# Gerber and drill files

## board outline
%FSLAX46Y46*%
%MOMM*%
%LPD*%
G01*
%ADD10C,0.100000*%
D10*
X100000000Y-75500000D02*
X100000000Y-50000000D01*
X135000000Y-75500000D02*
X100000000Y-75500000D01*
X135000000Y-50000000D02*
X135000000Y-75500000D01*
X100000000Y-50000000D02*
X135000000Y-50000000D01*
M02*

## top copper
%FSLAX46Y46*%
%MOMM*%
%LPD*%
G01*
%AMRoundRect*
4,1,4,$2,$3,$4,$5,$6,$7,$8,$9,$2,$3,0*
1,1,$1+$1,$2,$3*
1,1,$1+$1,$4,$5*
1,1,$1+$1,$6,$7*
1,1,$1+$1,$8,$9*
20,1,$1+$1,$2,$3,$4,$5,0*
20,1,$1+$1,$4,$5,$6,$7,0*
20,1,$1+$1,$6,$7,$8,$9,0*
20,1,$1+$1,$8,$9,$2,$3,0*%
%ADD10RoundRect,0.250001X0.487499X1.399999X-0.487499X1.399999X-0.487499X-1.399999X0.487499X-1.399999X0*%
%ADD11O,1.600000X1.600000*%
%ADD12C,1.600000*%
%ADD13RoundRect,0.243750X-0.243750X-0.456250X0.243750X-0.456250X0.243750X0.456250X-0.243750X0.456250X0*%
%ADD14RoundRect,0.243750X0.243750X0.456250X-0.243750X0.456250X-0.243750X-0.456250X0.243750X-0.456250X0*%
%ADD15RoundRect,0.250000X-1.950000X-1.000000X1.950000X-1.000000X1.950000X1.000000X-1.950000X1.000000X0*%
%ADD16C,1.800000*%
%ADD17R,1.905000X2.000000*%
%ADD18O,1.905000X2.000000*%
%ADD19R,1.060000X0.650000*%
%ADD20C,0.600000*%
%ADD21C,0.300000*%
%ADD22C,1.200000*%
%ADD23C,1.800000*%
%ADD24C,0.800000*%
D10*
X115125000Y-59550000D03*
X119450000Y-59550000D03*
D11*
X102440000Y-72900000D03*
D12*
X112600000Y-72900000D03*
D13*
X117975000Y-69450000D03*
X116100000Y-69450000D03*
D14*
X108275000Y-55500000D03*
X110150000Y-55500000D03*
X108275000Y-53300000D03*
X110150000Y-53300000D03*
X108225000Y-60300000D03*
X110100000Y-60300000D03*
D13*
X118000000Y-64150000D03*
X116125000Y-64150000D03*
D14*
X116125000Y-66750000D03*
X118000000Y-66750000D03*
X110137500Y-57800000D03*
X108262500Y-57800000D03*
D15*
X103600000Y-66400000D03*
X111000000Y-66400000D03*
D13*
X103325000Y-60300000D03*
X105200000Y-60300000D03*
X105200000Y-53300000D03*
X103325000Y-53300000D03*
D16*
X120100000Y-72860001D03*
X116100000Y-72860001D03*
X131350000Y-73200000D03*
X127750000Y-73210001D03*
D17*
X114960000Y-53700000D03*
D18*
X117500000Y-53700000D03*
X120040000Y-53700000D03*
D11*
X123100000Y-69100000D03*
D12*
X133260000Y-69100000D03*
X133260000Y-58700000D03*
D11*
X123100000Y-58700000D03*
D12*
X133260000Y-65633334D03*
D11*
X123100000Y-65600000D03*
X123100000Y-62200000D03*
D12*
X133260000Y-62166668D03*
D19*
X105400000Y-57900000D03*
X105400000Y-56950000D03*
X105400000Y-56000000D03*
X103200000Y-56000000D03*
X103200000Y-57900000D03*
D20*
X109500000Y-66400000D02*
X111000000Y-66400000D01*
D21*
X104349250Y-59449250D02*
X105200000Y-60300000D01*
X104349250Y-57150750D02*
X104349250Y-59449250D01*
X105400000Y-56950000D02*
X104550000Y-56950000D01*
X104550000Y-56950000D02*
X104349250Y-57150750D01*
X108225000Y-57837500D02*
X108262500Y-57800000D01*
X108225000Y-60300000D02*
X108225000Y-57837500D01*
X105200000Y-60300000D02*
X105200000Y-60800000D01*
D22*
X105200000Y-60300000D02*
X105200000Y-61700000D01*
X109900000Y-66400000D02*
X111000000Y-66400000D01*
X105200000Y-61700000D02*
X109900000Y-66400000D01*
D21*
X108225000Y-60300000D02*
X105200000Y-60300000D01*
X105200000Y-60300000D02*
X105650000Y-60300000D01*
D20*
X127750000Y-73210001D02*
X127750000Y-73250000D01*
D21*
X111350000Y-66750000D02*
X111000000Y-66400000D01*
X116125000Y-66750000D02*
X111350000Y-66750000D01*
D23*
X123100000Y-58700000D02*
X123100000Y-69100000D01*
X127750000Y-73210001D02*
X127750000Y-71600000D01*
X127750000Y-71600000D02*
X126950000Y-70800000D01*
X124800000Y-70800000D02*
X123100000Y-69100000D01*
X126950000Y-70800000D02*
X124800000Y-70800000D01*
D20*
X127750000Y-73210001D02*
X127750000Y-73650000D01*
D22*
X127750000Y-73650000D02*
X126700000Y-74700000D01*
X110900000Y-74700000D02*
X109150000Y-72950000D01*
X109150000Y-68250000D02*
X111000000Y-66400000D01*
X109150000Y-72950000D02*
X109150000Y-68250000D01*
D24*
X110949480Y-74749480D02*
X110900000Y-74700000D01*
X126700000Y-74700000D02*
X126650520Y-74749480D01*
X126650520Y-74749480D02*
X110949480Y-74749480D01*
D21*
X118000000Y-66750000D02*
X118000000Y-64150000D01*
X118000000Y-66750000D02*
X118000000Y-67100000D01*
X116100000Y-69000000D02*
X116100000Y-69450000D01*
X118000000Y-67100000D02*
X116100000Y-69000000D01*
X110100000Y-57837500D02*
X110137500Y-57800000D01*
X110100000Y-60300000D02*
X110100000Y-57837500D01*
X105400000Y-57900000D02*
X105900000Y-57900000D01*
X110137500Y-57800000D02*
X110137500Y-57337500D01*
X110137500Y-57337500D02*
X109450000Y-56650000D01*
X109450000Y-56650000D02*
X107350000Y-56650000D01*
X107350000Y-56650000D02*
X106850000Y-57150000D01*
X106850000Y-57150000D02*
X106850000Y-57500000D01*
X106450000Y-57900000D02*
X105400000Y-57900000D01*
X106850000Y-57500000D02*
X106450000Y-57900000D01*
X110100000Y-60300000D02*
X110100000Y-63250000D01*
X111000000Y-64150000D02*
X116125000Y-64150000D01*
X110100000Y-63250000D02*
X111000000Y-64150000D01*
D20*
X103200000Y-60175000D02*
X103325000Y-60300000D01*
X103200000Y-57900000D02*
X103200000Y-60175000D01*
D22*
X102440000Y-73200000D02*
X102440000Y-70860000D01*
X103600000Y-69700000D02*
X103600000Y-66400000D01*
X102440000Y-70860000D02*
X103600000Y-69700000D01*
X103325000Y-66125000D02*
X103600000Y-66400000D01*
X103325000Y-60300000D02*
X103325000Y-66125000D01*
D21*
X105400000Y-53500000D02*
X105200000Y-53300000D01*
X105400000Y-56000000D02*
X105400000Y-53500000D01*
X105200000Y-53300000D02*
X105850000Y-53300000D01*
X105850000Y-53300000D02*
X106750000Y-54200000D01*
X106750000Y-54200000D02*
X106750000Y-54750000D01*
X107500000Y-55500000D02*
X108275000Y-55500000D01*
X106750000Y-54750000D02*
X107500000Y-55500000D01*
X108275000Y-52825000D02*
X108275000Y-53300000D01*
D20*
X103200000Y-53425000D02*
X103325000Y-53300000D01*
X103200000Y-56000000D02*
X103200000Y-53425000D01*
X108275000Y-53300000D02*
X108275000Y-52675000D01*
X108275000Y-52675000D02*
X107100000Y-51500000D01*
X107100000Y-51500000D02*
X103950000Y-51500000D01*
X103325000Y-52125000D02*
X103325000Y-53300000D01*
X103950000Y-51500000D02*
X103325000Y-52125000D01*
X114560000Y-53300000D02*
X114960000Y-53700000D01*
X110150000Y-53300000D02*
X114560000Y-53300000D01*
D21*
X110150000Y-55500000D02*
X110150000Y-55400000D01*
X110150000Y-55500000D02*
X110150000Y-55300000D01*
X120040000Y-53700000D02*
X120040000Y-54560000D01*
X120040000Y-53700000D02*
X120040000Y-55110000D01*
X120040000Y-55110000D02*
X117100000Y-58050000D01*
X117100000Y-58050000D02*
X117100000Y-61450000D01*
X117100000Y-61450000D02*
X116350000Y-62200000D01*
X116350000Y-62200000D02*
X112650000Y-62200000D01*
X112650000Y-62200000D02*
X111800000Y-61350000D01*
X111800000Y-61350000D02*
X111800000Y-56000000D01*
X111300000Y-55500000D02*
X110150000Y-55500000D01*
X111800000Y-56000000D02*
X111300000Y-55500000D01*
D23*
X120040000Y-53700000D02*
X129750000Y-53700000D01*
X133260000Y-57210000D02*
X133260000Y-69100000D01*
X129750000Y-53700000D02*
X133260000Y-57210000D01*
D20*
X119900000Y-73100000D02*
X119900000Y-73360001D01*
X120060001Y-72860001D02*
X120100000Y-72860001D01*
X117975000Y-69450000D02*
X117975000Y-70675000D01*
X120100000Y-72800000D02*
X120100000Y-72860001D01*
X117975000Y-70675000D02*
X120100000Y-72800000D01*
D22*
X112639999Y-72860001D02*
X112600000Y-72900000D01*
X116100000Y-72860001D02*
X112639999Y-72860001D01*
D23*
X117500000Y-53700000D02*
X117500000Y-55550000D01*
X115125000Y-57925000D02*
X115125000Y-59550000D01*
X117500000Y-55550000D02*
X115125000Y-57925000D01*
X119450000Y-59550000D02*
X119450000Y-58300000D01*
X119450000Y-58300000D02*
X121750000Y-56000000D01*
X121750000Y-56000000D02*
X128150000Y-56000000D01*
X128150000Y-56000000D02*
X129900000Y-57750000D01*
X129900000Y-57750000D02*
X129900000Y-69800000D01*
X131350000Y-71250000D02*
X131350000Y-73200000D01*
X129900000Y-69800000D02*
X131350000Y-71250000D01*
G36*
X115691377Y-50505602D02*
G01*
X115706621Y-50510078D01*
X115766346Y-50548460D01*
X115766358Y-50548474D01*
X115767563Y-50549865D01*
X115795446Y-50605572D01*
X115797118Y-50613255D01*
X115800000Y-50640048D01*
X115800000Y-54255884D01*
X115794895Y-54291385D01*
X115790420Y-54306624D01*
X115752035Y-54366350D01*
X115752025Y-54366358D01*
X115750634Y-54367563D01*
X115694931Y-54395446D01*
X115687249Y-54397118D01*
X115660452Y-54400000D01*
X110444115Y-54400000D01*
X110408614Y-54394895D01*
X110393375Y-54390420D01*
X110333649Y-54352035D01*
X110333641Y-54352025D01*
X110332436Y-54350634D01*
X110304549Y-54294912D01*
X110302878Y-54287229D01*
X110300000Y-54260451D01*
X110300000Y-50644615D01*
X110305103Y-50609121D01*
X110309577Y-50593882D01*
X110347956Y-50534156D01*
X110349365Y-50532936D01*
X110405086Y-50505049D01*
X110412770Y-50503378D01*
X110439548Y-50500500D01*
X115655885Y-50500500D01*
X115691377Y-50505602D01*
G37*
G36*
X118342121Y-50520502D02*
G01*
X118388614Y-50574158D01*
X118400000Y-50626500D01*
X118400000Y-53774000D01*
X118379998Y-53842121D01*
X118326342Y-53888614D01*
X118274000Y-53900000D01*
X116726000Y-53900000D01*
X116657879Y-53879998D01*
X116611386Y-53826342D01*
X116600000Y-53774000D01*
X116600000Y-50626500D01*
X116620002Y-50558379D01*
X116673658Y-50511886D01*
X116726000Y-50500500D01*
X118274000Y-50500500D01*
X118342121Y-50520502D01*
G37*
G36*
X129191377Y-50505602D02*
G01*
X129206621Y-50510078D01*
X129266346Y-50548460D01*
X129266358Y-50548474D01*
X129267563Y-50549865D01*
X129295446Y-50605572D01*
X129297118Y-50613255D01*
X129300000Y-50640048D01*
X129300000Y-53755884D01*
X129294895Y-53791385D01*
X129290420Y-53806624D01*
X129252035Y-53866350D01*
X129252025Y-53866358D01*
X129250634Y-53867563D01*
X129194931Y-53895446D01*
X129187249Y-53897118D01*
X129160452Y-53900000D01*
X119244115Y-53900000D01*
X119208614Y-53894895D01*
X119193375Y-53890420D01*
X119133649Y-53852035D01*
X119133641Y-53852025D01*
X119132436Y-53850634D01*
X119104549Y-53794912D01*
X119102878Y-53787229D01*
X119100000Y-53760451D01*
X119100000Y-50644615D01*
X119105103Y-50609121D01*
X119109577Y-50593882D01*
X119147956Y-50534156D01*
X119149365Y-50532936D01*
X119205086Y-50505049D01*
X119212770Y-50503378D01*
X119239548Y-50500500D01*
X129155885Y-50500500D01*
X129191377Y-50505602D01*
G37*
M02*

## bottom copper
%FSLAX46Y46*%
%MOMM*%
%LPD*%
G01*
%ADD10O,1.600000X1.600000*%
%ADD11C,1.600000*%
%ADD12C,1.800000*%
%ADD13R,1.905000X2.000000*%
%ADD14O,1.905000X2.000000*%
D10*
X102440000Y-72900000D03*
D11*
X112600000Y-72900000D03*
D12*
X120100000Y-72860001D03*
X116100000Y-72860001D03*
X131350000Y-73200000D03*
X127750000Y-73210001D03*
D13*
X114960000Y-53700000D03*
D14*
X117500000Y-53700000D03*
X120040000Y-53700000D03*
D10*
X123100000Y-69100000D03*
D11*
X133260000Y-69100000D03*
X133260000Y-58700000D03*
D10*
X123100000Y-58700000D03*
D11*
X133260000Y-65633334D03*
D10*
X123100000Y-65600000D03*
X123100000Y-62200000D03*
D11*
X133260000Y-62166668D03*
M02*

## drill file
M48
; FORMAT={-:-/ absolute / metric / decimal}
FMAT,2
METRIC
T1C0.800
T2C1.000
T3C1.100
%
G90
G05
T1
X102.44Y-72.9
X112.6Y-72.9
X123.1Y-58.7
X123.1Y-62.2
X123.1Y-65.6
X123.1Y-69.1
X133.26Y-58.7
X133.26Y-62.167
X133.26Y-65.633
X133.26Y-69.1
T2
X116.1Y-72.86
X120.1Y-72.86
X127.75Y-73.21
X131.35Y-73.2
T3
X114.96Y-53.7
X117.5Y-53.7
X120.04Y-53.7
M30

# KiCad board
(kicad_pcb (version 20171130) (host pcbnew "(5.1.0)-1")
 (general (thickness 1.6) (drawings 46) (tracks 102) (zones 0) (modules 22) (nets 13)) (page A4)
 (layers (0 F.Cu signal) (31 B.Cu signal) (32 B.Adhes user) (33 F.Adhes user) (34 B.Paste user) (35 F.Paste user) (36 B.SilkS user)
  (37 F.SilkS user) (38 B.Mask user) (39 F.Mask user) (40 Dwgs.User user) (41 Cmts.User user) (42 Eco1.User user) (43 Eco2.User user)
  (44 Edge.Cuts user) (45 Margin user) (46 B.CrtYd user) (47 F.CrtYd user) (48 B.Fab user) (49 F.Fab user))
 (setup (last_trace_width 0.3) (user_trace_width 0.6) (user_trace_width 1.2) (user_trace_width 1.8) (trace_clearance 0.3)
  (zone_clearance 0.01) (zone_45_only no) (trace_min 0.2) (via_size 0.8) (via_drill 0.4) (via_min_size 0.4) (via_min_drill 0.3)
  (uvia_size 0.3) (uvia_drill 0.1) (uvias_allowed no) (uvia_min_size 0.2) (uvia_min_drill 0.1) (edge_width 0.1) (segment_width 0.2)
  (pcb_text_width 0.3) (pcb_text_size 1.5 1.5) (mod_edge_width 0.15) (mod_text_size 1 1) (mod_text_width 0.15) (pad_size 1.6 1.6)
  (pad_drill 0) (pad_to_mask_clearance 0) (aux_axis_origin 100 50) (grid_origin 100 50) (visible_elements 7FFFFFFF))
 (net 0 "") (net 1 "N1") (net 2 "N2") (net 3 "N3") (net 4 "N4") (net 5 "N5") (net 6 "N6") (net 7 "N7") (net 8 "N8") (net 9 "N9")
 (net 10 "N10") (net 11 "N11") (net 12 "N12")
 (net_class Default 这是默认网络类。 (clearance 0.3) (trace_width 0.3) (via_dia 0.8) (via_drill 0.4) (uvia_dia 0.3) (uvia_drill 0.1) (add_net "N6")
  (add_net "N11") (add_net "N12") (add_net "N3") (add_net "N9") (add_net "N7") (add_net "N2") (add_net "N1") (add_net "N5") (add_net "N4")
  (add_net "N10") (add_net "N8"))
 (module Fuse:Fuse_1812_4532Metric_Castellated (layer F.Cu) (at 117.2875 59.55 180)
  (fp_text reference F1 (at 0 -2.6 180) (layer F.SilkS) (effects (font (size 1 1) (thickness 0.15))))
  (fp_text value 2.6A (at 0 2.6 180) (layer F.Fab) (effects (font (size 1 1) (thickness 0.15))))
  (pad 2 smd roundrect (at 2.1625 0 180) (size 1.475 3.3) (layers F.Cu F.Paste F.Mask) (roundrect_rratio 0.169492) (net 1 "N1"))
  (pad 1 smd roundrect (at -2.1625 0 180) (size 1.475 3.3) (layers F.Cu F.Paste F.Mask) (roundrect_rratio 0.169492) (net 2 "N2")))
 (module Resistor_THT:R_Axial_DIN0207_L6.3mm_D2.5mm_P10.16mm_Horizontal (layer F.Cu) (at 112.6 72.9 180)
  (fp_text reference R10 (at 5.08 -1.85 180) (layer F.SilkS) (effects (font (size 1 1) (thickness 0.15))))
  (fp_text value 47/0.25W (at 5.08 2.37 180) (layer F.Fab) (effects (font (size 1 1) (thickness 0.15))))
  (pad 2 thru_hole oval (at 10.16 0 180) (size 1.6 1.6) (drill 0.8) (layers *.Cu *.Paste *.Mask) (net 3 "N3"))
  (pad 1 thru_hole circle (at 0 0 180) (size 1.6 1.6) (drill 0.8) (layers *.Cu *.Paste *.Mask) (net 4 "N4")))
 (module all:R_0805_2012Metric (layer F.Cu) (at 117.0375 69.45)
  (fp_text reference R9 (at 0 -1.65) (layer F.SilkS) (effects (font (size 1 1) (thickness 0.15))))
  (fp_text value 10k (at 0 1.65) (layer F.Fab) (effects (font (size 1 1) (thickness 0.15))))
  (pad 2 smd roundrect (at 0.9375 0) (size 0.975 1.4) (layers F.Cu F.Paste F.Mask) (roundrect_rratio 0.25) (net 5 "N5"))
  (pad 1 smd roundrect (at -0.9375 0) (size 0.975 1.4) (layers F.Cu F.Paste F.Mask) (roundrect_rratio 0.25) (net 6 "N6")))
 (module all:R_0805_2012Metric (layer F.Cu) (at 109.2125 55.5 180)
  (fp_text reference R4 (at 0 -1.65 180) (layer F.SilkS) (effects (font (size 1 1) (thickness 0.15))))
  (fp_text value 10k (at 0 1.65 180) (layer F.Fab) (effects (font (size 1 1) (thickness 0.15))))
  (pad 2 smd roundrect (at 0.9375 0 180) (size 0.975 1.4) (layers F.Cu F.Paste F.Mask) (roundrect_rratio 0.25) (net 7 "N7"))
  (pad 1 smd roundrect (at -0.9375 0 180) (size 0.975 1.4) (layers F.Cu F.Paste F.Mask) (roundrect_rratio 0.25) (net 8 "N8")))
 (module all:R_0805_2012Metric (layer F.Cu) (at 109.2125 53.3 180)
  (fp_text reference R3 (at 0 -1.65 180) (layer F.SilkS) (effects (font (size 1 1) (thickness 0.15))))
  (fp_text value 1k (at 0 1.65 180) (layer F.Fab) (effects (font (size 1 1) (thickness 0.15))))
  (pad 2 smd roundrect (at 0.9375 0 180) (size 0.975 1.4) (layers F.Cu F.Paste F.Mask) (roundrect_rratio 0.25) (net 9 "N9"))
  (pad 1 smd roundrect (at -0.9375 0 180) (size 0.975 1.4) (layers F.Cu F.Paste F.Mask) (roundrect_rratio 0.25) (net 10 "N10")))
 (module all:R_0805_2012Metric (layer F.Cu) (at 109.1625 60.3 180)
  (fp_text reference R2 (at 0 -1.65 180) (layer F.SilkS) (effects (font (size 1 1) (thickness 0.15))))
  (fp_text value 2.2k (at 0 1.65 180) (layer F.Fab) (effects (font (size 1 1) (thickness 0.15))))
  (pad 2 smd roundrect (at 0.9375 0 180) (size 0.975 1.4) (layers F.Cu F.Paste F.Mask) (roundrect_rratio 0.25) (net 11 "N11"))
  (pad 1 smd roundrect (at -0.9375 0 180) (size 0.975 1.4) (layers F.Cu F.Paste F.Mask) (roundrect_rratio 0.25) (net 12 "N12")))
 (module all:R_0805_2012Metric (layer F.Cu) (at 117.0625 64.15)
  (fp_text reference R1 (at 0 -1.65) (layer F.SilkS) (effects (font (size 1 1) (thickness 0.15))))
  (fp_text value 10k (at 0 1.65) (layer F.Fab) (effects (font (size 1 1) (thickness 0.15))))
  (pad 2 smd roundrect (at 0.9375 0) (size 0.975 1.4) (layers F.Cu F.Paste F.Mask) (roundrect_rratio 0.25) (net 6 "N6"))
  (pad 1 smd roundrect (at -0.9375 0) (size 0.975 1.4) (layers F.Cu F.Paste F.Mask) (roundrect_rratio 0.25) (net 12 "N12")))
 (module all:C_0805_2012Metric (layer F.Cu) (at 117.0625 66.75 180)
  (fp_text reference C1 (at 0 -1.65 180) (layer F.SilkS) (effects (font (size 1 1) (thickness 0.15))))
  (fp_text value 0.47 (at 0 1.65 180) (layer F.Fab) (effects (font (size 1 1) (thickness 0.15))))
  (pad 2 smd roundrect (at 0.9375 0 180) (size 0.975 1.4) (layers F.Cu F.Paste F.Mask) (roundrect_rratio 0.25) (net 11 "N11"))
  (pad 1 smd roundrect (at -0.9375 0 180) (size 0.975 1.4) (layers F.Cu F.Paste F.Mask) (roundrect_rratio 0.25) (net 6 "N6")))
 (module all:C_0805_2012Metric (layer F.Cu) (at 109.2 57.8 180)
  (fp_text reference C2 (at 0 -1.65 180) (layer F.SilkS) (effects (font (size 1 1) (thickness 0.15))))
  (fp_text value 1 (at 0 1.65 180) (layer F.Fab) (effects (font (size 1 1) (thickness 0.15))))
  (pad 1 smd roundrect (at -0.9375 0 180) (size 0.975 1.4) (layers F.Cu F.Paste F.Mask) (roundrect_rratio 0.25) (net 12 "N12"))
  (pad 2 smd roundrect (at 0.9375 0 180) (size 0.975 1.4) (layers F.Cu F.Paste F.Mask) (roundrect_rratio 0.25) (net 11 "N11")))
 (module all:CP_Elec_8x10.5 (layer F.Cu) (at 107.3 66.4)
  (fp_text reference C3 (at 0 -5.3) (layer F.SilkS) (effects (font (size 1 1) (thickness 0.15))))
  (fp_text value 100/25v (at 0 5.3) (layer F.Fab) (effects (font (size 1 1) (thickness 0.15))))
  (pad 1 smd roundrect (at -3.7 0) (size 4.4 2.5) (layers F.Cu F.Paste F.Mask) (roundrect_rratio 0.1) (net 3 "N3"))
  (pad 2 smd roundrect (at 3.7 0) (size 4.4 2.5) (layers F.Cu F.Paste F.Mask) (roundrect_rratio 0.1) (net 11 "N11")))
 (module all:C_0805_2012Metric (layer F.Cu) (at 104.2625 60.3)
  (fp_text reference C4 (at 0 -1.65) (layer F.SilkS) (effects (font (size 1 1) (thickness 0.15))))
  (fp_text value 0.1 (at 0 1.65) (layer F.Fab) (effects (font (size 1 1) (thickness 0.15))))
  (pad 1 smd roundrect (at -0.9375 0) (size 0.975 1.4) (layers F.Cu F.Paste F.Mask) (roundrect_rratio 0.25) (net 3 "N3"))
  (pad 2 smd roundrect (at 0.9375 0) (size 0.975 1.4) (layers F.Cu F.Paste F.Mask) (roundrect_rratio 0.25) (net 11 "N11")))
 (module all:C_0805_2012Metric (layer F.Cu) (at 104.2625 53.3)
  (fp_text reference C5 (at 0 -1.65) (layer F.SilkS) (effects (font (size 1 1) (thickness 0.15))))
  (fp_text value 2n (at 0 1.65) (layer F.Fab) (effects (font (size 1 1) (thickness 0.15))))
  (pad 2 smd roundrect (at 0.9375 0) (size 0.975 1.4) (layers F.Cu F.Paste F.Mask) (roundrect_rratio 0.25) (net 7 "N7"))
  (pad 1 smd roundrect (at -0.9375 0) (size 0.975 1.4) (layers F.Cu F.Paste F.Mask) (roundrect_rratio 0.25) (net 9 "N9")))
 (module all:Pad (layer F.Cu) (at 120.1 72.860001)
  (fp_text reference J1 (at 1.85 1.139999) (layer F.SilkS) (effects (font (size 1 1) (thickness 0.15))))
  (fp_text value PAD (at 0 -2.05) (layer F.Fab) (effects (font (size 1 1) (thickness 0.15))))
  (pad 1 thru_hole circle (at 0 0) (size 1.8 1.8) (drill 1) (layers *.Cu *.Paste *.Mask) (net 5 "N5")))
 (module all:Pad (layer F.Cu) (at 116.1 72.860001)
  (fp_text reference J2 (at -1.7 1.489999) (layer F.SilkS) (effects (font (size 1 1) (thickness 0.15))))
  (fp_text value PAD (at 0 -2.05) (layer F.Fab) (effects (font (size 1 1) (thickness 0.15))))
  (pad 1 thru_hole circle (at 0 0) (size 1.8 1.8) (drill 1) (layers *.Cu *.Paste *.Mask) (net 4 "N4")))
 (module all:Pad (layer F.Cu) (at 131.35 73.2)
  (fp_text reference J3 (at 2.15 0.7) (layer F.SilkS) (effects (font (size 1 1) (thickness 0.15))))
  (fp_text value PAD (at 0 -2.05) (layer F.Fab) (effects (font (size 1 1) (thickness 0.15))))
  (pad 1 thru_hole circle (at 0 0) (size 1.8 1.8) (drill 1) (layers *.Cu *.Paste *.Mask) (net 2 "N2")))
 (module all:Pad (layer F.Cu) (at 127.75 73.210001)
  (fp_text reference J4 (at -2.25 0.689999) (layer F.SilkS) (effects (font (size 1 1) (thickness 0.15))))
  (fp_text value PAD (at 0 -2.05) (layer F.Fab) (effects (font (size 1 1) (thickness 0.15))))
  (pad 1 thru_hole circle (at 0 0) (size 1.8 1.8) (drill 1) (layers *.Cu *.Paste *.Mask) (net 11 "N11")))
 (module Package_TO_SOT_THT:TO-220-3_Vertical (layer F.Cu) (at 114.96 53.7)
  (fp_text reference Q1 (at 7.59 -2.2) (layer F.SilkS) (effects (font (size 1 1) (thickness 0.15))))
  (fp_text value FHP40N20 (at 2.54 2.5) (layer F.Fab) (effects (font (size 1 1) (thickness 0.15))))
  (pad 1 thru_hole rect (at 0 0) (size 1.905 2) (drill 1.1) (layers *.Cu *.Paste *.Mask) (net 10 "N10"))
  (pad 2 thru_hole oval (at 2.54 0) (size 1.905 2) (drill 1.1) (layers *.Cu *.Paste *.Mask) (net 1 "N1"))
  (pad 3 thru_hole oval (at 5.08 0) (size 1.905 2) (drill 1.1) (layers *.Cu *.Paste *.Mask) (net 8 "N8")))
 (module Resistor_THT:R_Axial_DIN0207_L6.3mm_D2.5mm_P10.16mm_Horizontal (layer F.Cu) (at 133.26 69.1 180)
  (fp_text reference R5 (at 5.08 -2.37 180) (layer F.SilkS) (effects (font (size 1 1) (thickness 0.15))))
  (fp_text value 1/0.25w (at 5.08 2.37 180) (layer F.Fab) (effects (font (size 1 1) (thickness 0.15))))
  (pad 2 thru_hole oval (at 10.16 0 180) (size 1.6 1.6) (drill 0.8) (layers *.Cu *.Paste *.Mask) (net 11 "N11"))
  (pad 1 thru_hole circle (at 0 0 180) (size 1.6 1.6) (drill 0.8) (layers *.Cu *.Paste *.Mask) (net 8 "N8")))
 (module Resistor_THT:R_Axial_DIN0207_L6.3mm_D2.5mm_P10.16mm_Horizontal (layer F.Cu) (at 133.26 58.7 180)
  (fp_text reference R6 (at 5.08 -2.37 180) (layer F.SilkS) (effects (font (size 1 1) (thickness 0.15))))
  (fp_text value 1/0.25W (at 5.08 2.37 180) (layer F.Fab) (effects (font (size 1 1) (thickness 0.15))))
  (pad 1 thru_hole circle (at 0 0 180) (size 1.6 1.6) (drill 0.8) (layers *.Cu *.Paste *.Mask) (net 8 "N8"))
  (pad 2 thru_hole oval (at 10.16 0 180) (size 1.6 1.6) (drill 0.8) (layers *.Cu *.Paste *.Mask) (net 11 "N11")))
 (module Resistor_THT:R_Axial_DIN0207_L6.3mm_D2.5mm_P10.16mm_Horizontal (layer F.Cu) (at 133.26 65.6 180)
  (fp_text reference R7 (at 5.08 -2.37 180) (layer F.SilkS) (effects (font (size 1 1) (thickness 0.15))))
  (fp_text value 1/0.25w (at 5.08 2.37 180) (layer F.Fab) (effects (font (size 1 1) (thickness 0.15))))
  (pad 1 thru_hole circle (at 0 -0.033334 180) (size 1.6 1.6) (drill 0.8) (layers *.Cu *.Paste *.Mask) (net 8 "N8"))
  (pad 2 thru_hole oval (at 10.16 0 180) (size 1.6 1.6) (drill 0.8) (layers *.Cu *.Paste *.Mask) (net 11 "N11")))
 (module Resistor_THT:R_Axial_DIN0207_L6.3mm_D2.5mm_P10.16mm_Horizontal (layer F.Cu) (at 133.26 62.2 180)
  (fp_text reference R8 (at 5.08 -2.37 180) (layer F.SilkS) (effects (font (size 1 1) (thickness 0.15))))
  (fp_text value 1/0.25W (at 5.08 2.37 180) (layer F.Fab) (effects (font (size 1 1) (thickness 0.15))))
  (pad 2 thru_hole oval (at 10.16 0 180) (size 1.6 1.6) (drill 0.8) (layers *.Cu *.Paste *.Mask) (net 11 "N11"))
  (pad 1 thru_hole circle (at 0 0.033332 180) (size 1.6 1.6) (drill 0.8) (layers *.Cu *.Paste *.Mask) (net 8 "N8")))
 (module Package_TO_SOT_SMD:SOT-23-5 (layer F.Cu) (at 104.3 56.95 180)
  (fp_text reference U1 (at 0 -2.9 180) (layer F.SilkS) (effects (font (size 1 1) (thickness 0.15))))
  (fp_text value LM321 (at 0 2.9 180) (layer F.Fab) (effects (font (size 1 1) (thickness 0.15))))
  (pad 1 smd rect (at -1.1 -0.95 180) (size 1.06 0.65) (layers F.Cu F.Paste F.Mask) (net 12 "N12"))
  (pad 2 smd rect (at -1.1 0 180) (size 1.06 0.65) (layers F.Cu F.Paste F.Mask) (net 11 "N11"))
  (pad 3 smd rect (at -1.1 0.95 180) (size 1.06 0.65) (layers F.Cu F.Paste F.Mask) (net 7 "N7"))
  (pad 4 smd rect (at 1.1 0.95 180) (size 1.06 0.65) (layers F.Cu F.Paste F.Mask) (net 9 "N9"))
  (pad 5 smd rect (at 1.1 -0.95 180) (size 1.06 0.65) (layers F.Cu F.Paste F.Mask) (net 3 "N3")))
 (gr_line (start 100 75.5) (end 100 50) (layer Edge.Cuts) (width 0.1))
 (gr_line (start 135 75.5) (end 100 75.5) (layer Edge.Cuts) (width 0.1))
 (gr_line (start 135 50) (end 135 75.5) (layer Edge.Cuts) (width 0.1))
 (gr_line (start 100 50) (end 135 50) (layer Edge.Cuts) (width 0.1))
 (segment (start 109.5 66.4) (end 111 66.4) (width 0.6) (layer F.Cu) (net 11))
 (segment (start 104.34925 59.44925) (end 105.2 60.3) (width 0.3) (layer F.Cu) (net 11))
 (segment (start 104.34925 57.15075) (end 104.34925 59.44925) (width 0.3) (layer F.Cu) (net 11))
 (segment (start 105.4 56.95) (end 104.55 56.95) (width 0.3) (layer F.Cu) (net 11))
 (segment (start 104.55 56.95) (end 104.34925 57.15075) (width 0.3) (layer F.Cu) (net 11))
 (segment (start 108.225 57.8375) (end 108.2625 57.8) (width 0.3) (layer F.Cu) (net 11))
 (segment (start 108.225 60.3) (end 108.225 57.8375) (width 0.3) (layer F.Cu) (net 11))
 (segment (start 105.2 60.3) (end 105.2 60.8) (width 0.3) (layer F.Cu) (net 11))
 (segment (start 105.2 60.3) (end 105.2 61.7) (width 1.2) (layer F.Cu) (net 11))
 (segment (start 109.9 66.4) (end 111 66.4) (width 1.2) (layer F.Cu) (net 11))
 (segment (start 105.2 61.7) (end 109.9 66.4) (width 1.2) (layer F.Cu) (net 11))
 (segment (start 108.225 60.3) (end 105.2 60.3) (width 0.3) (layer F.Cu) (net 11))
 (segment (start 105.2 60.3) (end 105.65 60.3) (width 0.3) (layer F.Cu) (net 11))
 (segment (start 127.75 73.210001) (end 127.75 73.25) (width 0.6) (layer F.Cu) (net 11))
 (segment (start 111.35 66.75) (end 111 66.4) (width 0.3) (layer F.Cu) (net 11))
 (segment (start 116.125 66.75) (end 111.35 66.75) (width 0.3) (layer F.Cu) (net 11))
 (segment (start 123.1 58.7) (end 123.1 69.1) (width 1.8) (layer F.Cu) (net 11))
 (segment (start 127.75 73.210001) (end 127.75 71.6) (width 1.8) (layer F.Cu) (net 11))
 (segment (start 127.75 71.6) (end 126.95 70.8) (width 1.8) (layer F.Cu) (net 11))
 (segment (start 124.8 70.8) (end 123.1 69.1) (width 1.8) (layer F.Cu) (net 11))
 (segment (start 126.95 70.8) (end 124.8 70.8) (width 1.8) (layer F.Cu) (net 11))
 (segment (start 127.75 73.210001) (end 127.75 73.65) (width 0.6) (layer F.Cu) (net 11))
 (segment (start 127.75 73.65) (end 126.7 74.7) (width 1.2) (layer F.Cu) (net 11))
 (segment (start 110.9 74.7) (end 109.15 72.95) (width 1.2) (layer F.Cu) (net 11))
 (segment (start 109.15 68.25) (end 111 66.4) (width 1.2) (layer F.Cu) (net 11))
 (segment (start 109.15 72.95) (end 109.15 68.25) (width 1.2) (layer F.Cu) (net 11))
 (segment (start 110.94948 74.74948) (end 110.9 74.7) (width 0.8) (layer F.Cu) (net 11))
 (segment (start 126.7 74.7) (end 126.65052 74.74948) (width 0.8) (layer F.Cu) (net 11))
 (segment (start 126.65052 74.74948) (end 110.94948 74.74948) (width 0.8) (layer F.Cu) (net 11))
 (segment (start 118 66.75) (end 118 64.15) (width 0.3) (layer F.Cu) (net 6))
 (segment (start 118 66.75) (end 118 67.1) (width 0.3) (layer F.Cu) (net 6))
 (segment (start 116.1 69) (end 116.1 69.45) (width 0.3) (layer F.Cu) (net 6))
 (segment (start 118 67.1) (end 116.1 69) (width 0.3) (layer F.Cu) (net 6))
 (segment (start 110.1 57.8375) (end 110.1375 57.8) (width 0.3) (layer F.Cu) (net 12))
 (segment (start 110.1 60.3) (end 110.1 57.8375) (width 0.3) (layer F.Cu) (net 12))
 (segment (start 105.4 57.9) (end 105.9 57.9) (width 0.3) (layer F.Cu) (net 12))
 (segment (start 110.1375 57.8) (end 110.1375 57.3375) (width 0.3) (layer F.Cu) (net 12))
 (segment (start 110.1375 57.3375) (end 109.45 56.65) (width 0.3) (layer F.Cu) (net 12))
 (segment (start 109.45 56.65) (end 107.35 56.65) (width 0.3) (layer F.Cu) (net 12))
 (segment (start 107.35 56.65) (end 106.85 57.15) (width 0.3) (layer F.Cu) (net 12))
 (segment (start 106.85 57.15) (end 106.85 57.5) (width 0.3) (layer F.Cu) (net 12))
 (segment (start 106.45 57.9) (end 105.4 57.9) (width 0.3) (layer F.Cu) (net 12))
 (segment (start 106.85 57.5) (end 106.45 57.9) (width 0.3) (layer F.Cu) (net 12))
 (segment (start 110.1 60.3) (end 110.1 63.25) (width 0.3) (layer F.Cu) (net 12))
 (segment (start 111 64.15) (end 116.125 64.15) (width 0.3) (layer F.Cu) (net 12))
 (segment (start 110.1 63.25) (end 111 64.15) (width 0.3) (layer F.Cu) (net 12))
 (segment (start 103.2 60.175) (end 103.325 60.3) (width 0.6) (layer F.Cu) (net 3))
 (segment (start 103.2 57.9) (end 103.2 60.175) (width 0.6) (layer F.Cu) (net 3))
 (segment (start 102.44 73.2) (end 102.44 70.86) (width 1.2) (layer F.Cu) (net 3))
 (segment (start 103.6 69.7) (end 103.6 66.4) (width 1.2) (layer F.Cu) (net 3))
 (segment (start 102.44 70.86) (end 103.6 69.7) (width 1.2) (layer F.Cu) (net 3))
 (segment (start 103.325 66.125) (end 103.6 66.4) (width 1.2) (layer F.Cu) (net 3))
 (segment (start 103.325 60.3) (end 103.325 66.125) (width 1.2) (layer F.Cu) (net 3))
 (segment (start 105.4 53.5) (end 105.2 53.3) (width 0.3) (layer F.Cu) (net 7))
 (segment (start 105.4 56) (end 105.4 53.5) (width 0.3) (layer F.Cu) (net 7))
 (segment (start 105.2 53.3) (end 105.85 53.3) (width 0.3) (layer F.Cu) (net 7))
 (segment (start 105.85 53.3) (end 106.75 54.2) (width 0.3) (layer F.Cu) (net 7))
 (segment (start 106.75 54.2) (end 106.75 54.75) (width 0.3) (layer F.Cu) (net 7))
 (segment (start 107.5 55.5) (end 108.275 55.5) (width 0.3) (layer F.Cu) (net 7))
 (segment (start 106.75 54.75) (end 107.5 55.5) (width 0.3) (layer F.Cu) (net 7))
 (segment (start 108.275 52.825) (end 108.275 53.3) (width 0.3) (layer F.Cu) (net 9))
 (segment (start 103.2 53.425) (end 103.325 53.3) (width 0.6) (layer F.Cu) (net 9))
 (segment (start 103.2 56) (end 103.2 53.425) (width 0.6) (layer F.Cu) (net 9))
 (segment (start 108.275 53.3) (end 108.275 52.675) (width 0.6) (layer F.Cu) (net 9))
 (segment (start 108.275 52.675) (end 107.1 51.5) (width 0.6) (layer F.Cu) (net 9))
 (segment (start 107.1 51.5) (end 103.95 51.5) (width 0.6) (layer F.Cu) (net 9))
 (segment (start 103.325 52.125) (end 103.325 53.3) (width 0.6) (layer F.Cu) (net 9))
 (segment (start 103.95 51.5) (end 103.325 52.125) (width 0.6) (layer F.Cu) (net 9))
 (segment (start 114.56 53.3) (end 114.96 53.7) (width 0.6) (layer F.Cu) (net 10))
 (segment (start 110.15 53.3) (end 114.56 53.3) (width 0.6) (layer F.Cu) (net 10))
 (segment (start 110.15 55.5) (end 110.15 55.4) (width 0.3) (layer F.Cu) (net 8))
 (segment (start 110.15 55.5) (end 110.15 55.3) (width 0.3) (layer F.Cu) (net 8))
 (segment (start 120.04 53.7) (end 120.04 54.56) (width 0.3) (layer F.Cu) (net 8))
 (segment (start 120.04 53.7) (end 120.04 55.11) (width 0.3) (layer F.Cu) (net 8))
 (segment (start 120.04 55.11) (end 117.1 58.05) (width 0.3) (layer F.Cu) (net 8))
 (segment (start 117.1 58.05) (end 117.1 61.45) (width 0.3) (layer F.Cu) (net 8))
 (segment (start 117.1 61.45) (end 116.35 62.2) (width 0.3) (layer F.Cu) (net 8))
 (segment (start 116.35 62.2) (end 112.65 62.2) (width 0.3) (layer F.Cu) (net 8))
 (segment (start 112.65 62.2) (end 111.8 61.35) (width 0.3) (layer F.Cu) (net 8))
 (segment (start 111.8 61.35) (end 111.8 56) (width 0.3) (layer F.Cu) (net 8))
 (segment (start 111.3 55.5) (end 110.15 55.5) (width 0.3) (layer F.Cu) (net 8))
 (segment (start 111.8 56) (end 111.3 55.5) (width 0.3) (layer F.Cu) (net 8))
 (segment (start 120.04 53.7) (end 129.75 53.7) (width 1.8) (layer F.Cu) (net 8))
 (segment (start 133.26 57.21) (end 133.26 69.1) (width 1.8) (layer F.Cu) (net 8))
 (segment (start 129.75 53.7) (end 133.26 57.21) (width 1.8) (layer F.Cu) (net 8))
 (segment (start 119.9 73.1) (end 119.9 73.360001) (width 0.6) (layer F.Cu) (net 5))
 (segment (start 120.060001 72.860001) (end 120.1 72.860001) (width 0.6) (layer F.Cu) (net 5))
 (segment (start 117.975 69.45) (end 117.975 70.675) (width 0.6) (layer F.Cu) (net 5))
 (segment (start 120.1 72.8) (end 120.1 72.860001) (width 0.6) (layer F.Cu) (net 5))
 (segment (start 117.975 70.675) (end 120.1 72.8) (width 0.6) (layer F.Cu) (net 5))
 (segment (start 112.639999 72.860001) (end 112.6 72.9) (width 1.2) (layer F.Cu) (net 4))
 (segment (start 116.1 72.860001) (end 112.639999 72.860001) (width 1.2) (layer F.Cu) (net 4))
 (segment (start 117.5 53.7) (end 117.5 55.55) (width 1.8) (layer F.Cu) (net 1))
 (segment (start 115.125 57.925) (end 115.125 59.55) (width 1.8) (layer F.Cu) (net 1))
 (segment (start 117.5 55.55) (end 115.125 57.925) (width 1.8) (layer F.Cu) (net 1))
 (segment (start 119.45 59.55) (end 119.45 58.3) (width 1.8) (layer F.Cu) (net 2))
 (segment (start 119.45 58.3) (end 121.75 56) (width 1.8) (layer F.Cu) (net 2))
 (segment (start 121.75 56) (end 128.15 56) (width 1.8) (layer F.Cu) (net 2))
 (segment (start 128.15 56) (end 129.9 57.75) (width 1.8) (layer F.Cu) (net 2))
 (segment (start 129.9 57.75) (end 129.9 69.8) (width 1.8) (layer F.Cu) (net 2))
 (segment (start 131.35 71.25) (end 131.35 73.2) (width 1.8) (layer F.Cu) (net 2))
 (segment (start 129.9 69.8) (end 131.35 71.25) (width 1.8) (layer F.Cu) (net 2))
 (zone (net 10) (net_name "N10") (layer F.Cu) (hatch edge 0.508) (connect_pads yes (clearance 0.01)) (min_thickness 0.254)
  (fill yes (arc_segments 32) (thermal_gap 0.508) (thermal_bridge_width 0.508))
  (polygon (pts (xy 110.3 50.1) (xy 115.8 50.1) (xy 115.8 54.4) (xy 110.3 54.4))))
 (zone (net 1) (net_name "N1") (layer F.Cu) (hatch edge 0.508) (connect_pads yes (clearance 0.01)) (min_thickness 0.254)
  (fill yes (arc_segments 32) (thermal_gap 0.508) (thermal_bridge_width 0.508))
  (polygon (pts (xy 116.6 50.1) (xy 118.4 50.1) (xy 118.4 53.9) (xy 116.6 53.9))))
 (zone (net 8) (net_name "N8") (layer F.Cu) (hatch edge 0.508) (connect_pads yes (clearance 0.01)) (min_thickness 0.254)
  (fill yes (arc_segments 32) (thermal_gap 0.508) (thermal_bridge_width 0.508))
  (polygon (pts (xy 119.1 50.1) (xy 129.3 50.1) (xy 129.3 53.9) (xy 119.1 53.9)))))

